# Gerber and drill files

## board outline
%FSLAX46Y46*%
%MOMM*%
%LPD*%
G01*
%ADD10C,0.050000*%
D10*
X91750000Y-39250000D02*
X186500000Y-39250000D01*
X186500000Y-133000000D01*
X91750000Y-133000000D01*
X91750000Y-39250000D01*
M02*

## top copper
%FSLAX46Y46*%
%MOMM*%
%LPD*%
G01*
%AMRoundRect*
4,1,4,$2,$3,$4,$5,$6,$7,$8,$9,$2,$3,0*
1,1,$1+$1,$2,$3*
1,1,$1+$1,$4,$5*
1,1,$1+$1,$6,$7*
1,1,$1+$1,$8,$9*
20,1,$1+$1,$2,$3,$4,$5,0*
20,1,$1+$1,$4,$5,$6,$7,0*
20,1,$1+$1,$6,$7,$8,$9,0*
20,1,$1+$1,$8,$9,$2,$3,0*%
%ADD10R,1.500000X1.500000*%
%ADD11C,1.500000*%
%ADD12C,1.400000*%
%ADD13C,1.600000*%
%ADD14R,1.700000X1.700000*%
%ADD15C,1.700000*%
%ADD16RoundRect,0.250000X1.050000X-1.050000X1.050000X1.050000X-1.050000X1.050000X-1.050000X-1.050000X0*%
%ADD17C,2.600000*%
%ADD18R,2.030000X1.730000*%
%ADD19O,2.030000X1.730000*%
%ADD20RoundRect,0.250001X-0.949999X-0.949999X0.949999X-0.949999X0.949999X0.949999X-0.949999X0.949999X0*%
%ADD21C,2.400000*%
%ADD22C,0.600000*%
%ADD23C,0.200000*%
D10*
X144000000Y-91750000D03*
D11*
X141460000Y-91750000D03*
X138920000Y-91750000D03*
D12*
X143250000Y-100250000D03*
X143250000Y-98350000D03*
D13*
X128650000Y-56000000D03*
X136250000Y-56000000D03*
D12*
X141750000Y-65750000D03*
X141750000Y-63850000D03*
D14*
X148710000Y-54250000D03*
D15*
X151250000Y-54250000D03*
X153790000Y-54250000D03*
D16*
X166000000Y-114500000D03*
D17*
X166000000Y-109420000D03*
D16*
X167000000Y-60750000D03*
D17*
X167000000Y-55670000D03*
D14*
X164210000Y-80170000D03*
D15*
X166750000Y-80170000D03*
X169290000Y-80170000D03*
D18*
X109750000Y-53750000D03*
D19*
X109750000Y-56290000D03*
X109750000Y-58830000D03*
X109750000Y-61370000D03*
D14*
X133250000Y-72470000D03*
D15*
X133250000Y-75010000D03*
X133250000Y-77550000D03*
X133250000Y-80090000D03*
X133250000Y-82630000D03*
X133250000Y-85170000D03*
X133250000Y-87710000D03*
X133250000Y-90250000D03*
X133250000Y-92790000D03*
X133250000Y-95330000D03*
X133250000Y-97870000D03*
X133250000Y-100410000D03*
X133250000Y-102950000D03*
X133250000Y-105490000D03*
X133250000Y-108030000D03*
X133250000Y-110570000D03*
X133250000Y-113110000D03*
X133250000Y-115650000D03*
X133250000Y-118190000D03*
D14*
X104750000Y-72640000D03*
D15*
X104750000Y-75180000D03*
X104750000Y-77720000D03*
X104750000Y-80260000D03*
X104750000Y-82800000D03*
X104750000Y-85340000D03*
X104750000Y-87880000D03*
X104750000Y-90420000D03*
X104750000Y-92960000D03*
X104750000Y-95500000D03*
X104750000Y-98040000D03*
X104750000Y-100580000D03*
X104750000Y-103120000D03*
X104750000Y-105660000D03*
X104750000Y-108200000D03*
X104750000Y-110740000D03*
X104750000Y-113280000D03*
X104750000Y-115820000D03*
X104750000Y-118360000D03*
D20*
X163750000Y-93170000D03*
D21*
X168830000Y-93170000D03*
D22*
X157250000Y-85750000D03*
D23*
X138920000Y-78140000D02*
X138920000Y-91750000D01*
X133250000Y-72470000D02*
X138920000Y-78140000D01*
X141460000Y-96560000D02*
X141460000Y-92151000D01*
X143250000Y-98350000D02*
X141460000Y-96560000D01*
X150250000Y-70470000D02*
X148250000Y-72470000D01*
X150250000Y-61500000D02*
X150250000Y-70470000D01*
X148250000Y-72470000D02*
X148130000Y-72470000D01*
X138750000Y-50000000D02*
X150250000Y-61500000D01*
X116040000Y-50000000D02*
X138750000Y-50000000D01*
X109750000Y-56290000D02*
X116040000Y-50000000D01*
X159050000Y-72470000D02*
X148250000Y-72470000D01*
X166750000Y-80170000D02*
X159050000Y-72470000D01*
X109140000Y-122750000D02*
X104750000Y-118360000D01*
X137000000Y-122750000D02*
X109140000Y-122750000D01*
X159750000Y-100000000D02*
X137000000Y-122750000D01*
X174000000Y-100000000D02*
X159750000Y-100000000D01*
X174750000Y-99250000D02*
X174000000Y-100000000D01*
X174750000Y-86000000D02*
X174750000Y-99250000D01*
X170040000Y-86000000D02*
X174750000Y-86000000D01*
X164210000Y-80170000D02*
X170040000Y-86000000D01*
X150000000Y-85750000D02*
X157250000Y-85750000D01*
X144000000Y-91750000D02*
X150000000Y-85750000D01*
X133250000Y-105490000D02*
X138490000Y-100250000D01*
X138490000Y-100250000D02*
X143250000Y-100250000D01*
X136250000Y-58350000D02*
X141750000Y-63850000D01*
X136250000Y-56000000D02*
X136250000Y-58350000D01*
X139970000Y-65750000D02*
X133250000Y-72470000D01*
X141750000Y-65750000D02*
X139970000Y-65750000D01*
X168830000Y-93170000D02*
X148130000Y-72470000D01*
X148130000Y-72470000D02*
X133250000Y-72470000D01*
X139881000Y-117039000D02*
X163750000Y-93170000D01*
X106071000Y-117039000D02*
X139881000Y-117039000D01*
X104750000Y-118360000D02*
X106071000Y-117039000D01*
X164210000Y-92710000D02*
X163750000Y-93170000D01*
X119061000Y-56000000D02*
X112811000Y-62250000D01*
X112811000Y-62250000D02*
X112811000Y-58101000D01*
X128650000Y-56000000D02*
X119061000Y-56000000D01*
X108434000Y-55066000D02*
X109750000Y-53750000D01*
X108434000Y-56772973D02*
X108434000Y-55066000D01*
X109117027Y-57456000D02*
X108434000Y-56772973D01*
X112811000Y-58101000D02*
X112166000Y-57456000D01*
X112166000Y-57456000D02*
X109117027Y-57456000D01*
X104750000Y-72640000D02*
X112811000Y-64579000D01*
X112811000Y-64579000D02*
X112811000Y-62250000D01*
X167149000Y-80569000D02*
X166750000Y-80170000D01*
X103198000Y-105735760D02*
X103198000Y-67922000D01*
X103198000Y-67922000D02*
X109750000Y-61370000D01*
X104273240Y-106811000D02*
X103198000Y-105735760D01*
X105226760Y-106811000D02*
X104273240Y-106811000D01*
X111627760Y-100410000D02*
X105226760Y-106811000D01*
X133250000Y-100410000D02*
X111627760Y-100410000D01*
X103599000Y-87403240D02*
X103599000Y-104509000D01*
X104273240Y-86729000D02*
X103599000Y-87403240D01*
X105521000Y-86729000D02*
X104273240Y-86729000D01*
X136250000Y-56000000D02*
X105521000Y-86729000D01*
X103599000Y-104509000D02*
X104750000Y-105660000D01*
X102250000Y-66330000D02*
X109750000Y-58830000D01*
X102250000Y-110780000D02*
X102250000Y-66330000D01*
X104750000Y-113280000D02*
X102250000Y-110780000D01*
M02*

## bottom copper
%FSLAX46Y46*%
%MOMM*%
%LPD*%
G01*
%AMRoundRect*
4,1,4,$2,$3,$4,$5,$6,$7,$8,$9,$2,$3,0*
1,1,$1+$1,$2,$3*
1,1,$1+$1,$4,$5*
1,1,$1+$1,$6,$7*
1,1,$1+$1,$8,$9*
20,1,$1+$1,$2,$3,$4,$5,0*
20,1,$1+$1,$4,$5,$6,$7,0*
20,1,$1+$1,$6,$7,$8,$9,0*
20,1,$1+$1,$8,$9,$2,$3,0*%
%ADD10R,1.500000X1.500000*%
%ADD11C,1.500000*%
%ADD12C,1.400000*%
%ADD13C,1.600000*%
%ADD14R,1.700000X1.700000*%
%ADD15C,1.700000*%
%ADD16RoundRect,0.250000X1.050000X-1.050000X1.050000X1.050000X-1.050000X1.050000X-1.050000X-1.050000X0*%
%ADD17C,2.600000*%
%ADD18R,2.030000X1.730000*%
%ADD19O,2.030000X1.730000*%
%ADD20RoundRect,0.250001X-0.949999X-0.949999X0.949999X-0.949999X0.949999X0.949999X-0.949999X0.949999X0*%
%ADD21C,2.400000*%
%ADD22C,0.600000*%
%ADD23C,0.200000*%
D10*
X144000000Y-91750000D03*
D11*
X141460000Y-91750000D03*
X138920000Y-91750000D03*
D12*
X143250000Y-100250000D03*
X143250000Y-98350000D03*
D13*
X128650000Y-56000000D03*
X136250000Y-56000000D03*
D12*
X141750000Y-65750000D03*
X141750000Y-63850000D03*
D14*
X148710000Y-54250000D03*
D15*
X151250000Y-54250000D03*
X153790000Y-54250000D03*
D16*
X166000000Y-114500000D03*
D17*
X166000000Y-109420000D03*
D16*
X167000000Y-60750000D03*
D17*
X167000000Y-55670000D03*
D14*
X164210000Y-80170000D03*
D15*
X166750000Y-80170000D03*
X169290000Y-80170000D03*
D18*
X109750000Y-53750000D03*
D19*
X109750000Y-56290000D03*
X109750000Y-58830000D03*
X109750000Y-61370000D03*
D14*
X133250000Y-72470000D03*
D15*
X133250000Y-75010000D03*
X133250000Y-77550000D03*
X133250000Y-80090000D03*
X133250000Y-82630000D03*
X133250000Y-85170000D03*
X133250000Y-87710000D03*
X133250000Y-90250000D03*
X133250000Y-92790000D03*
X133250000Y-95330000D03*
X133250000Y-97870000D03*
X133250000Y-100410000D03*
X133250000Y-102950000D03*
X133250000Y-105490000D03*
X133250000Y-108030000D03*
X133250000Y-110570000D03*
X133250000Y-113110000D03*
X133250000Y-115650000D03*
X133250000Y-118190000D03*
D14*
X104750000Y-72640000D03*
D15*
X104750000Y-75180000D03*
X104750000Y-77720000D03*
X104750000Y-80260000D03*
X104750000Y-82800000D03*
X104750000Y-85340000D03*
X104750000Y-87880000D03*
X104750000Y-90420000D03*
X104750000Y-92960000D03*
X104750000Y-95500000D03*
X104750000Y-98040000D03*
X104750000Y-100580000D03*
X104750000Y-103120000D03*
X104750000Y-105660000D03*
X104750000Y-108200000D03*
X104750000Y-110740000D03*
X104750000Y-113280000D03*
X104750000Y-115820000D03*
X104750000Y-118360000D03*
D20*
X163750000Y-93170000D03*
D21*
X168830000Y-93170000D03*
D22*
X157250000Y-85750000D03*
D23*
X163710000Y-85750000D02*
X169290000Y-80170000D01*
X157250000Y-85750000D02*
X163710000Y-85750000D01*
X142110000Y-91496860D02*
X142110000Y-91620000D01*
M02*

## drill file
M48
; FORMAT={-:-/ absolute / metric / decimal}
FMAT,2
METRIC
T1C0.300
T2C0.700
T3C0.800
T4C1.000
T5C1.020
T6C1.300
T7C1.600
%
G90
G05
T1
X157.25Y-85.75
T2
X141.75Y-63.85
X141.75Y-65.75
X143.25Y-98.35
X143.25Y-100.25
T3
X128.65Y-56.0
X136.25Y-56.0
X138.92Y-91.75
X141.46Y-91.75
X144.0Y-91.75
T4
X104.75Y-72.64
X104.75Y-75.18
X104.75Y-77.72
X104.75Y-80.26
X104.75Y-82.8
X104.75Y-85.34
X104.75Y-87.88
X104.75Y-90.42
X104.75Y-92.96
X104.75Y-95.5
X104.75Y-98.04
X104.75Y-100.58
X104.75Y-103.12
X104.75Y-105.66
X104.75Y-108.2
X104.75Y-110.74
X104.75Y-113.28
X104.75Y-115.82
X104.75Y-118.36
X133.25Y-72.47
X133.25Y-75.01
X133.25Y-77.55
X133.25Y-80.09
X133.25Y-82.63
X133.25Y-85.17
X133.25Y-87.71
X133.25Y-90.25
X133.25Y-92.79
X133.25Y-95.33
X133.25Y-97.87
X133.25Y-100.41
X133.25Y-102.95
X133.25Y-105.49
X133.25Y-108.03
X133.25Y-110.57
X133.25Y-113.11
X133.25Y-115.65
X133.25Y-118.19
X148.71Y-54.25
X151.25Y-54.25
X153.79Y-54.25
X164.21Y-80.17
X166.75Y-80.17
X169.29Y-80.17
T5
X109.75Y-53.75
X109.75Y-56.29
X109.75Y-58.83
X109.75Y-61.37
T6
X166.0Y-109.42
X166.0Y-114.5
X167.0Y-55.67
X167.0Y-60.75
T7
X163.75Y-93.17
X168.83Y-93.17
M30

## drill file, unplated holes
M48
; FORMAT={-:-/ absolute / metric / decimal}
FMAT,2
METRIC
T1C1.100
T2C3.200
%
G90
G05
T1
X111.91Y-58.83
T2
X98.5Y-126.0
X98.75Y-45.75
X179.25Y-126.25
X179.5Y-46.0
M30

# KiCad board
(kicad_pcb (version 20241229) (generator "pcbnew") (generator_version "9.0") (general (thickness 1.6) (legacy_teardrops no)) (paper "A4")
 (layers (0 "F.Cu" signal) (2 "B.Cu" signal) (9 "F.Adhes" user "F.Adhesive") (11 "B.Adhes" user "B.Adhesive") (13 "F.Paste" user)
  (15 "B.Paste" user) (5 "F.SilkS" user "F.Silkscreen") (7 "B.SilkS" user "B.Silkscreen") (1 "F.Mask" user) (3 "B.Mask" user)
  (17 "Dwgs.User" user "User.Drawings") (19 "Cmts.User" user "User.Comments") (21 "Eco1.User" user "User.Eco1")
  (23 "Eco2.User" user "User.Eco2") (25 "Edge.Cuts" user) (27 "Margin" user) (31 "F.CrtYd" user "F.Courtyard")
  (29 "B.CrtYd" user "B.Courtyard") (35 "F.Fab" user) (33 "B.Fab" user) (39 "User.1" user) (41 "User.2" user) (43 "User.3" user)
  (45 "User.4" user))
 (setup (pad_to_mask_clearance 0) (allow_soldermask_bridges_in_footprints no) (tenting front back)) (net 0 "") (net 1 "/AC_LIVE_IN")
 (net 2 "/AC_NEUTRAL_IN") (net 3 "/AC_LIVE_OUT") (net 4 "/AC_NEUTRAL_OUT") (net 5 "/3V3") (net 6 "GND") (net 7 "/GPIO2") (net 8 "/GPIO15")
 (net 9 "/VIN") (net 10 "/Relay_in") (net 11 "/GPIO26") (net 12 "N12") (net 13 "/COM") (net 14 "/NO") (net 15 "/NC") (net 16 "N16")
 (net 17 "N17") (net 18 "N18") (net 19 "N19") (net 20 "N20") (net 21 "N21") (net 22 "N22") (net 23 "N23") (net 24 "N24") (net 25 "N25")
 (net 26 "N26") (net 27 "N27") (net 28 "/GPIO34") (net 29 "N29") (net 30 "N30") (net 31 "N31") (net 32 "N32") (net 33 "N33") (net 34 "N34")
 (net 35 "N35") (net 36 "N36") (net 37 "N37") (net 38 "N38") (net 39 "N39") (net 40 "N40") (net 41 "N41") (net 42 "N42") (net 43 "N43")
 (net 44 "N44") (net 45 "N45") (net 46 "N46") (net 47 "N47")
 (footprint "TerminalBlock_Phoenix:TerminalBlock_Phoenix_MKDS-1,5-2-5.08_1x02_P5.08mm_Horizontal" (layer "F.Cu") (at 167 60.75 90)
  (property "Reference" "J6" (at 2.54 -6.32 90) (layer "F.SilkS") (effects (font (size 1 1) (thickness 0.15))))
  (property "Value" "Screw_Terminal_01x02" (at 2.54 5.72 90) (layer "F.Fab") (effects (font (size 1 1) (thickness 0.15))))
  (pad "1" thru_hole roundrect (at 0 0 90) (size 2.6 2.6) (drill 1.3) (layers "*.Cu" "*.Mask") (remove_unused_layers no)
   (roundrect_rratio 0.096154) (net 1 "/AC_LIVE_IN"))
  (pad "2" thru_hole circle (at 5.08 0 90) (size 2.6 2.6) (drill 1.3) (layers "*.Cu" "*.Mask") (remove_unused_layers no)
   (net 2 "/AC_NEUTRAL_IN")))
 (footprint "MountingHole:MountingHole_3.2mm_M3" (layer "F.Cu") (at 179.25 126.25)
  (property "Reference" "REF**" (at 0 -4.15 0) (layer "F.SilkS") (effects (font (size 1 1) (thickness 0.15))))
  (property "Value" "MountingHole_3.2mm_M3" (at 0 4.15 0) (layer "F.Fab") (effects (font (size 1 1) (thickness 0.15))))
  (pad "" np_thru_hole circle (at 0 0) (size 3.2 3.2) (drill 3.2) (layers "*.Cu" "*.Mask")))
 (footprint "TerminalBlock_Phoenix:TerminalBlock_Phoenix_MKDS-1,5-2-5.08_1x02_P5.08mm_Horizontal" (layer "F.Cu") (at 166 114.5 90)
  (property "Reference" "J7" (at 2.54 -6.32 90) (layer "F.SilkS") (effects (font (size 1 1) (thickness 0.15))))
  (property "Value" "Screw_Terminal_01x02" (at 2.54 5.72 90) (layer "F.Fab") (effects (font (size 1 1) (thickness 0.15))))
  (pad "1" thru_hole roundrect (at 0 0 90) (size 2.6 2.6) (drill 1.3) (layers "*.Cu" "*.Mask") (remove_unused_layers no)
   (roundrect_rratio 0.096154) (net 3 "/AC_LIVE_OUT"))
  (pad "2" thru_hole circle (at 5.08 0 90) (size 2.6 2.6) (drill 1.3) (layers "*.Cu" "*.Mask") (remove_unused_layers no)
   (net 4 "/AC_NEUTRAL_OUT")))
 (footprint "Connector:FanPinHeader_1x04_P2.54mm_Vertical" (layer "F.Cu") (at 109.75 53.75 -90)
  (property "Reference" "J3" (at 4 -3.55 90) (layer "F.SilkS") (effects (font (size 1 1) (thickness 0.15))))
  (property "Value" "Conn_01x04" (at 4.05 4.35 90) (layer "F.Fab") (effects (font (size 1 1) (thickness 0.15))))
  (pad "" np_thru_hole circle (at 5.08 -2.16) (size 1.1 1.1) (drill 1.1) (layers "*.Cu" "*.Mask"))
  (pad "1" thru_hole rect (at 0 0) (size 2.03 1.73) (drill 1.02) (layers "*.Cu" "*.Mask") (remove_unused_layers no) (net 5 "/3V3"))
  (pad "2" thru_hole oval (at 2.54 0) (size 2.03 1.73) (drill 1.02) (layers "*.Cu" "*.Mask") (remove_unused_layers no) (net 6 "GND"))
  (pad "3" thru_hole oval (at 5.08 0) (size 2.03 1.73) (drill 1.02) (layers "*.Cu" "*.Mask") (remove_unused_layers no) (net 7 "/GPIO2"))
  (pad "4" thru_hole oval (at 7.62 0) (size 2.03 1.73) (drill 1.02) (layers "*.Cu" "*.Mask") (remove_unused_layers no) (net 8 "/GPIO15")))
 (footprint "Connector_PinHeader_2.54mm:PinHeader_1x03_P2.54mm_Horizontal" (layer "F.Cu") (at 164.21 80.17 90)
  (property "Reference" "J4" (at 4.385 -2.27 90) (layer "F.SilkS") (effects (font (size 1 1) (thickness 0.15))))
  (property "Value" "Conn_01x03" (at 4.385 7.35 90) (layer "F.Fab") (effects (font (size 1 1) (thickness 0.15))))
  (pad "1" thru_hole rect (at 0 0 90) (size 1.7 1.7) (drill 1) (layers "*.Cu" "*.Mask") (remove_unused_layers no) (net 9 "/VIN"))
  (pad "2" thru_hole circle (at 0 2.54 90) (size 1.7 1.7) (drill 1) (layers "*.Cu" "*.Mask") (remove_unused_layers no) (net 6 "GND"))
  (pad "3" thru_hole circle (at 0 5.08 90) (size 1.7 1.7) (drill 1) (layers "*.Cu" "*.Mask") (remove_unused_layers no) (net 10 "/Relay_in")))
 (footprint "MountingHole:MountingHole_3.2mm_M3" (layer "F.Cu") (at 98.75 45.75)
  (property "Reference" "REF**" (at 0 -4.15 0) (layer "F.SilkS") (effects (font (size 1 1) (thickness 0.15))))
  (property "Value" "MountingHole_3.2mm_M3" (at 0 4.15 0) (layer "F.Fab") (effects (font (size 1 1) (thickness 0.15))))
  (pad "" np_thru_hole circle (at 0 0) (size 3.2 3.2) (drill 3.2) (layers "*.Cu" "*.Mask")))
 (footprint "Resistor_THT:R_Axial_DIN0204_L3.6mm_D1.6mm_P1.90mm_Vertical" (layer "F.Cu") (at 143.25 100.25 90)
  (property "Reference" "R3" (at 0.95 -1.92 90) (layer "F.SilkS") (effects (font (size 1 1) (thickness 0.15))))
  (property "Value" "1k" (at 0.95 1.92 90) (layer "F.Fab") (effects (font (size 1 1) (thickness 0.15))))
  (pad "1" thru_hole circle (at 0 0 90) (size 1.4 1.4) (drill 0.7) (layers "*.Cu" "*.Mask") (remove_unused_layers no) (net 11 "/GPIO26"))
  (pad "2" thru_hole circle (at 1.9 0 90) (size 1.4 1.4) (drill 0.7) (layers "*.Cu" "*.Mask") (remove_unused_layers no) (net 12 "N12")))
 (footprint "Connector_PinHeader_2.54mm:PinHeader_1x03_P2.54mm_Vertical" (layer "F.Cu") (at 148.71 54.25 90)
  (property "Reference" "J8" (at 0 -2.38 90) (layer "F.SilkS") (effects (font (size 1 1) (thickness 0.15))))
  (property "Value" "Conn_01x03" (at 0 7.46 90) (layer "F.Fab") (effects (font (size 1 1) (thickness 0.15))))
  (pad "1" thru_hole rect (at 0 0 90) (size 1.7 1.7) (drill 1) (layers "*.Cu" "*.Mask") (remove_unused_layers no) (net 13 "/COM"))
  (pad "2" thru_hole circle (at 0 2.54 90) (size 1.7 1.7) (drill 1) (layers "*.Cu" "*.Mask") (remove_unused_layers no) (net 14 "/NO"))
  (pad "3" thru_hole circle (at 0 5.08 90) (size 1.7 1.7) (drill 1) (layers "*.Cu" "*.Mask") (remove_unused_layers no) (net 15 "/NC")))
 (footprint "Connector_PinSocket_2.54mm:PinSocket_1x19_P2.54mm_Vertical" (layer "F.Cu") (at 104.75 72.64)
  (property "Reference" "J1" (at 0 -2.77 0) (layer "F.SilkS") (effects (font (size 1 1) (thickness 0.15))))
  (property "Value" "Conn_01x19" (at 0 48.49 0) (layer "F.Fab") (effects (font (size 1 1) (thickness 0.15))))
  (pad "1" thru_hole rect (at 0 0) (size 1.7 1.7) (drill 1) (layers "*.Cu" "*.Mask") (remove_unused_layers no) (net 5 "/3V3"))
  (pad "2" thru_hole circle (at 0 2.54) (size 1.7 1.7) (drill 1) (layers "*.Cu" "*.Mask") (remove_unused_layers no) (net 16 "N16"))
  (pad "3" thru_hole circle (at 0 5.08) (size 1.7 1.7) (drill 1) (layers "*.Cu" "*.Mask") (remove_unused_layers no) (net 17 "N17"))
  (pad "4" thru_hole circle (at 0 7.62) (size 1.7 1.7) (drill 1) (layers "*.Cu" "*.Mask") (remove_unused_layers no) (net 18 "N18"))
  (pad "5" thru_hole circle (at 0 10.16) (size 1.7 1.7) (drill 1) (layers "*.Cu" "*.Mask") (remove_unused_layers no) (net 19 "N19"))
  (pad "6" thru_hole circle (at 0 12.7) (size 1.7 1.7) (drill 1) (layers "*.Cu" "*.Mask") (remove_unused_layers no) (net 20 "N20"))
  (pad "7" thru_hole circle (at 0 15.24) (size 1.7 1.7) (drill 1) (layers "*.Cu" "*.Mask") (remove_unused_layers no) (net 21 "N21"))
  (pad "8" thru_hole circle (at 0 17.78) (size 1.7 1.7) (drill 1) (layers "*.Cu" "*.Mask") (remove_unused_layers no) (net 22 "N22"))
  (pad "9" thru_hole circle (at 0 20.32) (size 1.7 1.7) (drill 1) (layers "*.Cu" "*.Mask") (remove_unused_layers no) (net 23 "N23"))
  (pad "10" thru_hole circle (at 0 22.86) (size 1.7 1.7) (drill 1) (layers "*.Cu" "*.Mask") (remove_unused_layers no) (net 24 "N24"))
  (pad "11" thru_hole circle (at 0 25.4) (size 1.7 1.7) (drill 1) (layers "*.Cu" "*.Mask") (remove_unused_layers no) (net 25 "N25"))
  (pad "12" thru_hole circle (at 0 27.94) (size 1.7 1.7) (drill 1) (layers "*.Cu" "*.Mask") (remove_unused_layers no) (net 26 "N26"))
  (pad "13" thru_hole circle (at 0 30.48) (size 1.7 1.7) (drill 1) (layers "*.Cu" "*.Mask") (remove_unused_layers no) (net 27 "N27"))
  (pad "14" thru_hole circle (at 0 33.02) (size 1.7 1.7) (drill 1) (layers "*.Cu" "*.Mask") (remove_unused_layers no) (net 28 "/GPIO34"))
  (pad "15" thru_hole circle (at 0 35.56) (size 1.7 1.7) (drill 1) (layers "*.Cu" "*.Mask") (remove_unused_layers no) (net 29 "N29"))
  (pad "16" thru_hole circle (at 0 38.1) (size 1.7 1.7) (drill 1) (layers "*.Cu" "*.Mask") (remove_unused_layers no) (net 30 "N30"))
  (pad "17" thru_hole circle (at 0 40.64) (size 1.7 1.7) (drill 1) (layers "*.Cu" "*.Mask") (remove_unused_layers no) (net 7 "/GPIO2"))
  (pad "18" thru_hole circle (at 0 43.18) (size 1.7 1.7) (drill 1) (layers "*.Cu" "*.Mask") (remove_unused_layers no) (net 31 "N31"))
  (pad "19" thru_hole circle (at 0 45.72) (size 1.7 1.7) (drill 1) (layers "*.Cu" "*.Mask") (remove_unused_layers no) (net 9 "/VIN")))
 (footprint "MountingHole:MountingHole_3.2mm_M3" (layer "F.Cu") (at 98.5 126)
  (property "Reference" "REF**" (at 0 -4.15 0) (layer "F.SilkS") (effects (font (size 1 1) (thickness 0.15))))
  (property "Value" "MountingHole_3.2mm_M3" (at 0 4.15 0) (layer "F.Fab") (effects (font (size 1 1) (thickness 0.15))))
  (pad "" np_thru_hole circle (at 0 0) (size 3.2 3.2) (drill 3.2) (layers "*.Cu" "*.Mask")))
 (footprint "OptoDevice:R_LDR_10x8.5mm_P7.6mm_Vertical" (layer "F.Cu") (at 128.65 56)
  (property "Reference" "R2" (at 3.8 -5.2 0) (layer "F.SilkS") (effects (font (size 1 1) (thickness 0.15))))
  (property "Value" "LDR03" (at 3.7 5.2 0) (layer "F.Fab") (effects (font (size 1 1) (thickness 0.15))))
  (pad "1" thru_hole circle (at 0 0) (size 1.6 1.6) (drill 0.8) (layers "*.Cu" "*.Mask") (remove_unused_layers no) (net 5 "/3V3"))
  (pad "2" thru_hole circle (at 7.6 0) (size 1.6 1.6) (drill 0.8) (layers "*.Cu" "*.Mask") (remove_unused_layers no) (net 28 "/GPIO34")))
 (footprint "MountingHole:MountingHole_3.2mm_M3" (layer "F.Cu") (at 179.5 46)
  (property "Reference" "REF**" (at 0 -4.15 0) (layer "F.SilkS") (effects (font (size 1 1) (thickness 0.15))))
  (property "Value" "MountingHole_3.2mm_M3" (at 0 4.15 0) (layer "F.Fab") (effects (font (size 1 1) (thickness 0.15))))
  (pad "" np_thru_hole circle (at 0 0) (size 3.2 3.2) (drill 3.2) (layers "*.Cu" "*.Mask")))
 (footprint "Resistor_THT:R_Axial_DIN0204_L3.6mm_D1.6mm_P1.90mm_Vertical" (layer "F.Cu") (at 141.75 65.75 90)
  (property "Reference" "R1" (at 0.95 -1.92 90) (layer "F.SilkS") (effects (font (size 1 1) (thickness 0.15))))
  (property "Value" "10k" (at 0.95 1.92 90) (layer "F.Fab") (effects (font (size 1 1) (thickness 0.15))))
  (pad "1" thru_hole circle (at 0 0 90) (size 1.4 1.4) (drill 0.7) (layers "*.Cu" "*.Mask") (remove_unused_layers no) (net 6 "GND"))
  (pad "2" thru_hole circle (at 1.9 0 90) (size 1.4 1.4) (drill 0.7) (layers "*.Cu" "*.Mask") (remove_unused_layers no) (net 28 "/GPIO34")))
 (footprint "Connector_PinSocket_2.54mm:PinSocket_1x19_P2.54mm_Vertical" (layer "F.Cu") (at 133.25 72.47)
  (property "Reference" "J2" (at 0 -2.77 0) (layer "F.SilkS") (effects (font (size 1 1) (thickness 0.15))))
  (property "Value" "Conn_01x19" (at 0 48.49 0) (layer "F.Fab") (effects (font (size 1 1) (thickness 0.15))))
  (pad "1" thru_hole rect (at 0 0) (size 1.7 1.7) (drill 1) (layers "*.Cu" "*.Mask") (remove_unused_layers no) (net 6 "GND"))
  (pad "2" thru_hole circle (at 0 2.54) (size 1.7 1.7) (drill 1) (layers "*.Cu" "*.Mask") (remove_unused_layers no) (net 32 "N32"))
  (pad "3" thru_hole circle (at 0 5.08) (size 1.7 1.7) (drill 1) (layers "*.Cu" "*.Mask") (remove_unused_layers no) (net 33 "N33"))
  (pad "4" thru_hole circle (at 0 7.62) (size 1.7 1.7) (drill 1) (layers "*.Cu" "*.Mask") (remove_unused_layers no) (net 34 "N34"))
  (pad "5" thru_hole circle (at 0 10.16) (size 1.7 1.7) (drill 1) (layers "*.Cu" "*.Mask") (remove_unused_layers no) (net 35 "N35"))
  (pad "6" thru_hole circle (at 0 12.7) (size 1.7 1.7) (drill 1) (layers "*.Cu" "*.Mask") (remove_unused_layers no) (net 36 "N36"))
  (pad "7" thru_hole circle (at 0 15.24) (size 1.7 1.7) (drill 1) (layers "*.Cu" "*.Mask") (remove_unused_layers no) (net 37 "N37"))
  (pad "8" thru_hole circle (at 0 17.78) (size 1.7 1.7) (drill 1) (layers "*.Cu" "*.Mask") (remove_unused_layers no) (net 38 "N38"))
  (pad "9" thru_hole circle (at 0 20.32) (size 1.7 1.7) (drill 1) (layers "*.Cu" "*.Mask") (remove_unused_layers no) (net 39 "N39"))
  (pad "10" thru_hole circle (at 0 22.86) (size 1.7 1.7) (drill 1) (layers "*.Cu" "*.Mask") (remove_unused_layers no) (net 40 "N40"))
  (pad "11" thru_hole circle (at 0 25.4) (size 1.7 1.7) (drill 1) (layers "*.Cu" "*.Mask") (remove_unused_layers no) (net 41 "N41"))
  (pad "12" thru_hole circle (at 0 27.94) (size 1.7 1.7) (drill 1) (layers "*.Cu" "*.Mask") (remove_unused_layers no) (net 8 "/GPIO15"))
  (pad "13" thru_hole circle (at 0 30.48) (size 1.7 1.7) (drill 1) (layers "*.Cu" "*.Mask") (remove_unused_layers no) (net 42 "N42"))
  (pad "14" thru_hole circle (at 0 33.02) (size 1.7 1.7) (drill 1) (layers "*.Cu" "*.Mask") (remove_unused_layers no) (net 11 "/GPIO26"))
  (pad "15" thru_hole circle (at 0 35.56) (size 1.7 1.7) (drill 1) (layers "*.Cu" "*.Mask") (remove_unused_layers no) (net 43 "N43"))
  (pad "16" thru_hole circle (at 0 38.1) (size 1.7 1.7) (drill 1) (layers "*.Cu" "*.Mask") (remove_unused_layers no) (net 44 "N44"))
  (pad "17" thru_hole circle (at 0 40.64) (size 1.7 1.7) (drill 1) (layers "*.Cu" "*.Mask") (remove_unused_layers no) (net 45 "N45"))
  (pad "18" thru_hole circle (at 0 43.18) (size 1.7 1.7) (drill 1) (layers "*.Cu" "*.Mask") (remove_unused_layers no) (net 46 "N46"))
  (pad "19" thru_hole circle (at 0 45.72) (size 1.7 1.7) (drill 1) (layers "*.Cu" "*.Mask") (remove_unused_layers no) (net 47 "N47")))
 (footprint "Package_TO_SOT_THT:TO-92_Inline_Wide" (layer "B.Cu") (at 144 91.75 180)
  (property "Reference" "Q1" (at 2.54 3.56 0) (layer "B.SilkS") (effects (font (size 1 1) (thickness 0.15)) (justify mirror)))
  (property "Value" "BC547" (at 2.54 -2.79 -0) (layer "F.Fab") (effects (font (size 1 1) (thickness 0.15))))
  (pad "1" thru_hole rect (at 0 0 180) (size 1.5 1.5) (drill 0.8) (layers "*.Cu" "*.Mask") (remove_unused_layers no) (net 10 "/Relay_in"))
  (pad "2" thru_hole circle (at 2.54 0 180) (size 1.5 1.5) (drill 0.8) (layers "*.Cu" "*.Mask") (remove_unused_layers no) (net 12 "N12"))
  (pad "3" thru_hole circle (at 5.08 0 180) (size 1.5 1.5) (drill 0.8) (layers "*.Cu" "*.Mask") (remove_unused_layers no) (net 6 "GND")))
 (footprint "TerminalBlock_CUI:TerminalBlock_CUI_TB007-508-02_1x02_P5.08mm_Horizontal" (layer "B.Cu") (at 163.75 93.17)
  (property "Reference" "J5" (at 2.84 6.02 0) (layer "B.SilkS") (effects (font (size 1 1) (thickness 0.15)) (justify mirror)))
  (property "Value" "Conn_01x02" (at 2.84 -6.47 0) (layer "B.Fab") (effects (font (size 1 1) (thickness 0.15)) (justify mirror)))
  (pad "1" thru_hole roundrect (at 0 0) (size 2.4 2.4) (drill 1.6) (layers "*.Cu" "*.Mask") (remove_unused_layers no)
   (roundrect_rratio 0.104167) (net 9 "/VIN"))
  (pad "2" thru_hole circle (at 5.08 0) (size 2.4 2.4) (drill 1.6) (layers "*.Cu" "*.Mask") (remove_unused_layers no) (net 6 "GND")))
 (gr_rect (start 91.75 39.25) (end 186.5 133) (stroke (width 0.05) (type default)) (fill no) (layer "Edge.Cuts"))
 (segment (start 104.27324 86.729) (end 103.599 87.40324) (width 0.2) (layer "F.Cu") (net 28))
 (segment (start 103.599 104.509) (end 104.75 105.66) (width 0.2) (layer "F.Cu") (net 28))
 (segment (start 105.521 86.729) (end 104.27324 86.729) (width 0.2) (layer "F.Cu") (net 28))
 (segment (start 136.25 56) (end 105.521 86.729) (width 0.2) (layer "F.Cu") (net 28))
 (segment (start 103.599 87.40324) (end 103.599 104.509) (width 0.2) (layer "F.Cu") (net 28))
 (segment (start 136.25 58.35) (end 141.75 63.85) (width 0.2) (layer "F.Cu") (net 28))
 (segment (start 136.25 56) (end 136.25 58.35) (width 0.2) (layer "F.Cu") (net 28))
 (segment (start 112.166 57.456) (end 109.117027 57.456) (width 0.2) (layer "F.Cu") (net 5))
 (segment (start 112.811 64.579) (end 112.811 62.25) (width 0.2) (layer "F.Cu") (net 5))
 (segment (start 119.061 56) (end 112.811 62.25) (width 0.2) (layer "F.Cu") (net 5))
 (segment (start 112.811 62.25) (end 112.811 58.101) (width 0.2) (layer "F.Cu") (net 5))
 (segment (start 108.434 56.772973) (end 108.434 55.066) (width 0.2) (layer "F.Cu") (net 5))
 (segment (start 112.811 58.101) (end 112.166 57.456) (width 0.2) (layer "F.Cu") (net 5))
 (segment (start 109.117027 57.456) (end 108.434 56.772973) (width 0.2) (layer "F.Cu") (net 5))
 (segment (start 128.65 56) (end 119.061 56) (width 0.2) (layer "F.Cu") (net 5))
 (segment (start 108.434 55.066) (end 109.75 53.75) (width 0.2) (layer "F.Cu") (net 5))
 (segment (start 104.75 72.64) (end 112.811 64.579) (width 0.2) (layer "F.Cu") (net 5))
 (segment (start 164.21 80.17) (end 170.04 86) (width 0.2) (layer "F.Cu") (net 9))
 (segment (start 137 122.75) (end 109.14 122.75) (width 0.2) (layer "F.Cu") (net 9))
 (segment (start 174 100) (end 159.75 100) (width 0.2) (layer "F.Cu") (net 9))
 (segment (start 139.881 117.039) (end 163.75 93.17) (width 0.2) (layer "F.Cu") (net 9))
 (segment (start 170.04 86) (end 174.75 86) (width 0.2) (layer "F.Cu") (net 9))
 (segment (start 109.14 122.75) (end 104.75 118.36) (width 0.2) (layer "F.Cu") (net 9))
 (segment (start 174.75 99.25) (end 174 100) (width 0.2) (layer "F.Cu") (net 9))
 (segment (start 106.071 117.039) (end 139.881 117.039) (width 0.2) (layer "F.Cu") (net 9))
 (segment (start 164.21 92.71) (end 163.75 93.17) (width 0.2) (layer "F.Cu") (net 9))
 (segment (start 159.75 100) (end 137 122.75) (width 0.2) (layer "F.Cu") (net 9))
 (segment (start 104.75 118.36) (end 106.071 117.039) (width 0.2) (layer "F.Cu") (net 9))
 (segment (start 174.75 86) (end 174.75 99.25) (width 0.2) (layer "F.Cu") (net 9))
 (segment (start 102.25 110.78) (end 102.25 66.33) (width 0.2) (layer "F.Cu") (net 7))
 (segment (start 102.25 66.33) (end 109.75 58.83) (width 0.2) (layer "F.Cu") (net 7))
 (segment (start 104.75 113.28) (end 102.25 110.78) (width 0.2) (layer "F.Cu") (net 7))
 (segment (start 141.75 65.75) (end 139.97 65.75) (width 0.2) (layer "F.Cu") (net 6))
 (segment (start 150.25 70.47) (end 148.25 72.47) (width 0.2) (layer "F.Cu") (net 6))
 (segment (start 168.83 93.17) (end 148.13 72.47) (width 0.2) (layer "F.Cu") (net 6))
 (segment (start 139.97 65.75) (end 133.25 72.47) (width 0.2) (layer "F.Cu") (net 6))
 (segment (start 167.149 80.569) (end 166.75 80.17) (width 0.2) (layer "F.Cu") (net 6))
 (segment (start 148.25 72.47) (end 148.13 72.47) (width 0.2) (layer "F.Cu") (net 6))
 (segment (start 138.75 50) (end 150.25 61.5) (width 0.2) (layer "F.Cu") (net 6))
 (segment (start 109.75 56.29) (end 116.04 50) (width 0.2) (layer "F.Cu") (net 6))
 (segment (start 166.75 80.17) (end 159.05 72.47) (width 0.2) (layer "F.Cu") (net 6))
 (segment (start 148.13 72.47) (end 133.25 72.47) (width 0.2) (layer "F.Cu") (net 6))
 (segment (start 116.04 50) (end 138.75 50) (width 0.2) (layer "F.Cu") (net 6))
 (segment (start 150.25 61.5) (end 150.25 70.47) (width 0.2) (layer "F.Cu") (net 6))
 (segment (start 138.92 78.14) (end 138.92 91.75) (width 0.2) (layer "F.Cu") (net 6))
 (segment (start 159.05 72.47) (end 148.25 72.47) (width 0.2) (layer "F.Cu") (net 6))
 (segment (start 133.25 72.47) (end 138.92 78.14) (width 0.2) (layer "F.Cu") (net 6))
 (segment (start 133.25 100.41) (end 111.62776 100.41) (width 0.2) (layer "F.Cu") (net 8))
 (segment (start 103.198 105.73576) (end 103.198 67.922) (width 0.2) (layer "F.Cu") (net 8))
 (segment (start 104.27324 106.811) (end 103.198 105.73576) (width 0.2) (layer "F.Cu") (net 8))
 (segment (start 103.198 67.922) (end 109.75 61.37) (width 0.2) (layer "F.Cu") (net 8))
 (segment (start 111.62776 100.41) (end 105.22676 106.811) (width 0.2) (layer "F.Cu") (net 8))
 (segment (start 105.22676 106.811) (end 104.27324 106.811) (width 0.2) (layer "F.Cu") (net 8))
 (segment (start 133.25 105.49) (end 138.49 100.25) (width 0.2) (layer "F.Cu") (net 11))
 (segment (start 138.49 100.25) (end 143.25 100.25) (width 0.2) (layer "F.Cu") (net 11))
 (segment (start 150 85.75) (end 157.25 85.75) (width 0.2) (layer "F.Cu") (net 10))
 (segment (start 144 91.75) (end 150 85.75) (width 0.2) (layer "F.Cu") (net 10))
 (via (at 157.25 85.75) (size 0.6) (drill 0.3) (layers "F.Cu" "B.Cu") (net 10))
 (segment (start 157.25 85.75) (end 163.71 85.75) (width 0.2) (layer "B.Cu") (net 10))
 (segment (start 163.71 85.75) (end 169.29 80.17) (width 0.2) (layer "B.Cu") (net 10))
 (segment (start 141.46 96.56) (end 141.46 92.151) (width 0.2) (layer "F.Cu") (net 12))
 (segment (start 143.25 98.35) (end 141.46 96.56) (width 0.2) (layer "F.Cu") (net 12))
 (segment (start 142.11 91.49686) (end 142.11 91.62) (width 0.2) (layer "B.Cu") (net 12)))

